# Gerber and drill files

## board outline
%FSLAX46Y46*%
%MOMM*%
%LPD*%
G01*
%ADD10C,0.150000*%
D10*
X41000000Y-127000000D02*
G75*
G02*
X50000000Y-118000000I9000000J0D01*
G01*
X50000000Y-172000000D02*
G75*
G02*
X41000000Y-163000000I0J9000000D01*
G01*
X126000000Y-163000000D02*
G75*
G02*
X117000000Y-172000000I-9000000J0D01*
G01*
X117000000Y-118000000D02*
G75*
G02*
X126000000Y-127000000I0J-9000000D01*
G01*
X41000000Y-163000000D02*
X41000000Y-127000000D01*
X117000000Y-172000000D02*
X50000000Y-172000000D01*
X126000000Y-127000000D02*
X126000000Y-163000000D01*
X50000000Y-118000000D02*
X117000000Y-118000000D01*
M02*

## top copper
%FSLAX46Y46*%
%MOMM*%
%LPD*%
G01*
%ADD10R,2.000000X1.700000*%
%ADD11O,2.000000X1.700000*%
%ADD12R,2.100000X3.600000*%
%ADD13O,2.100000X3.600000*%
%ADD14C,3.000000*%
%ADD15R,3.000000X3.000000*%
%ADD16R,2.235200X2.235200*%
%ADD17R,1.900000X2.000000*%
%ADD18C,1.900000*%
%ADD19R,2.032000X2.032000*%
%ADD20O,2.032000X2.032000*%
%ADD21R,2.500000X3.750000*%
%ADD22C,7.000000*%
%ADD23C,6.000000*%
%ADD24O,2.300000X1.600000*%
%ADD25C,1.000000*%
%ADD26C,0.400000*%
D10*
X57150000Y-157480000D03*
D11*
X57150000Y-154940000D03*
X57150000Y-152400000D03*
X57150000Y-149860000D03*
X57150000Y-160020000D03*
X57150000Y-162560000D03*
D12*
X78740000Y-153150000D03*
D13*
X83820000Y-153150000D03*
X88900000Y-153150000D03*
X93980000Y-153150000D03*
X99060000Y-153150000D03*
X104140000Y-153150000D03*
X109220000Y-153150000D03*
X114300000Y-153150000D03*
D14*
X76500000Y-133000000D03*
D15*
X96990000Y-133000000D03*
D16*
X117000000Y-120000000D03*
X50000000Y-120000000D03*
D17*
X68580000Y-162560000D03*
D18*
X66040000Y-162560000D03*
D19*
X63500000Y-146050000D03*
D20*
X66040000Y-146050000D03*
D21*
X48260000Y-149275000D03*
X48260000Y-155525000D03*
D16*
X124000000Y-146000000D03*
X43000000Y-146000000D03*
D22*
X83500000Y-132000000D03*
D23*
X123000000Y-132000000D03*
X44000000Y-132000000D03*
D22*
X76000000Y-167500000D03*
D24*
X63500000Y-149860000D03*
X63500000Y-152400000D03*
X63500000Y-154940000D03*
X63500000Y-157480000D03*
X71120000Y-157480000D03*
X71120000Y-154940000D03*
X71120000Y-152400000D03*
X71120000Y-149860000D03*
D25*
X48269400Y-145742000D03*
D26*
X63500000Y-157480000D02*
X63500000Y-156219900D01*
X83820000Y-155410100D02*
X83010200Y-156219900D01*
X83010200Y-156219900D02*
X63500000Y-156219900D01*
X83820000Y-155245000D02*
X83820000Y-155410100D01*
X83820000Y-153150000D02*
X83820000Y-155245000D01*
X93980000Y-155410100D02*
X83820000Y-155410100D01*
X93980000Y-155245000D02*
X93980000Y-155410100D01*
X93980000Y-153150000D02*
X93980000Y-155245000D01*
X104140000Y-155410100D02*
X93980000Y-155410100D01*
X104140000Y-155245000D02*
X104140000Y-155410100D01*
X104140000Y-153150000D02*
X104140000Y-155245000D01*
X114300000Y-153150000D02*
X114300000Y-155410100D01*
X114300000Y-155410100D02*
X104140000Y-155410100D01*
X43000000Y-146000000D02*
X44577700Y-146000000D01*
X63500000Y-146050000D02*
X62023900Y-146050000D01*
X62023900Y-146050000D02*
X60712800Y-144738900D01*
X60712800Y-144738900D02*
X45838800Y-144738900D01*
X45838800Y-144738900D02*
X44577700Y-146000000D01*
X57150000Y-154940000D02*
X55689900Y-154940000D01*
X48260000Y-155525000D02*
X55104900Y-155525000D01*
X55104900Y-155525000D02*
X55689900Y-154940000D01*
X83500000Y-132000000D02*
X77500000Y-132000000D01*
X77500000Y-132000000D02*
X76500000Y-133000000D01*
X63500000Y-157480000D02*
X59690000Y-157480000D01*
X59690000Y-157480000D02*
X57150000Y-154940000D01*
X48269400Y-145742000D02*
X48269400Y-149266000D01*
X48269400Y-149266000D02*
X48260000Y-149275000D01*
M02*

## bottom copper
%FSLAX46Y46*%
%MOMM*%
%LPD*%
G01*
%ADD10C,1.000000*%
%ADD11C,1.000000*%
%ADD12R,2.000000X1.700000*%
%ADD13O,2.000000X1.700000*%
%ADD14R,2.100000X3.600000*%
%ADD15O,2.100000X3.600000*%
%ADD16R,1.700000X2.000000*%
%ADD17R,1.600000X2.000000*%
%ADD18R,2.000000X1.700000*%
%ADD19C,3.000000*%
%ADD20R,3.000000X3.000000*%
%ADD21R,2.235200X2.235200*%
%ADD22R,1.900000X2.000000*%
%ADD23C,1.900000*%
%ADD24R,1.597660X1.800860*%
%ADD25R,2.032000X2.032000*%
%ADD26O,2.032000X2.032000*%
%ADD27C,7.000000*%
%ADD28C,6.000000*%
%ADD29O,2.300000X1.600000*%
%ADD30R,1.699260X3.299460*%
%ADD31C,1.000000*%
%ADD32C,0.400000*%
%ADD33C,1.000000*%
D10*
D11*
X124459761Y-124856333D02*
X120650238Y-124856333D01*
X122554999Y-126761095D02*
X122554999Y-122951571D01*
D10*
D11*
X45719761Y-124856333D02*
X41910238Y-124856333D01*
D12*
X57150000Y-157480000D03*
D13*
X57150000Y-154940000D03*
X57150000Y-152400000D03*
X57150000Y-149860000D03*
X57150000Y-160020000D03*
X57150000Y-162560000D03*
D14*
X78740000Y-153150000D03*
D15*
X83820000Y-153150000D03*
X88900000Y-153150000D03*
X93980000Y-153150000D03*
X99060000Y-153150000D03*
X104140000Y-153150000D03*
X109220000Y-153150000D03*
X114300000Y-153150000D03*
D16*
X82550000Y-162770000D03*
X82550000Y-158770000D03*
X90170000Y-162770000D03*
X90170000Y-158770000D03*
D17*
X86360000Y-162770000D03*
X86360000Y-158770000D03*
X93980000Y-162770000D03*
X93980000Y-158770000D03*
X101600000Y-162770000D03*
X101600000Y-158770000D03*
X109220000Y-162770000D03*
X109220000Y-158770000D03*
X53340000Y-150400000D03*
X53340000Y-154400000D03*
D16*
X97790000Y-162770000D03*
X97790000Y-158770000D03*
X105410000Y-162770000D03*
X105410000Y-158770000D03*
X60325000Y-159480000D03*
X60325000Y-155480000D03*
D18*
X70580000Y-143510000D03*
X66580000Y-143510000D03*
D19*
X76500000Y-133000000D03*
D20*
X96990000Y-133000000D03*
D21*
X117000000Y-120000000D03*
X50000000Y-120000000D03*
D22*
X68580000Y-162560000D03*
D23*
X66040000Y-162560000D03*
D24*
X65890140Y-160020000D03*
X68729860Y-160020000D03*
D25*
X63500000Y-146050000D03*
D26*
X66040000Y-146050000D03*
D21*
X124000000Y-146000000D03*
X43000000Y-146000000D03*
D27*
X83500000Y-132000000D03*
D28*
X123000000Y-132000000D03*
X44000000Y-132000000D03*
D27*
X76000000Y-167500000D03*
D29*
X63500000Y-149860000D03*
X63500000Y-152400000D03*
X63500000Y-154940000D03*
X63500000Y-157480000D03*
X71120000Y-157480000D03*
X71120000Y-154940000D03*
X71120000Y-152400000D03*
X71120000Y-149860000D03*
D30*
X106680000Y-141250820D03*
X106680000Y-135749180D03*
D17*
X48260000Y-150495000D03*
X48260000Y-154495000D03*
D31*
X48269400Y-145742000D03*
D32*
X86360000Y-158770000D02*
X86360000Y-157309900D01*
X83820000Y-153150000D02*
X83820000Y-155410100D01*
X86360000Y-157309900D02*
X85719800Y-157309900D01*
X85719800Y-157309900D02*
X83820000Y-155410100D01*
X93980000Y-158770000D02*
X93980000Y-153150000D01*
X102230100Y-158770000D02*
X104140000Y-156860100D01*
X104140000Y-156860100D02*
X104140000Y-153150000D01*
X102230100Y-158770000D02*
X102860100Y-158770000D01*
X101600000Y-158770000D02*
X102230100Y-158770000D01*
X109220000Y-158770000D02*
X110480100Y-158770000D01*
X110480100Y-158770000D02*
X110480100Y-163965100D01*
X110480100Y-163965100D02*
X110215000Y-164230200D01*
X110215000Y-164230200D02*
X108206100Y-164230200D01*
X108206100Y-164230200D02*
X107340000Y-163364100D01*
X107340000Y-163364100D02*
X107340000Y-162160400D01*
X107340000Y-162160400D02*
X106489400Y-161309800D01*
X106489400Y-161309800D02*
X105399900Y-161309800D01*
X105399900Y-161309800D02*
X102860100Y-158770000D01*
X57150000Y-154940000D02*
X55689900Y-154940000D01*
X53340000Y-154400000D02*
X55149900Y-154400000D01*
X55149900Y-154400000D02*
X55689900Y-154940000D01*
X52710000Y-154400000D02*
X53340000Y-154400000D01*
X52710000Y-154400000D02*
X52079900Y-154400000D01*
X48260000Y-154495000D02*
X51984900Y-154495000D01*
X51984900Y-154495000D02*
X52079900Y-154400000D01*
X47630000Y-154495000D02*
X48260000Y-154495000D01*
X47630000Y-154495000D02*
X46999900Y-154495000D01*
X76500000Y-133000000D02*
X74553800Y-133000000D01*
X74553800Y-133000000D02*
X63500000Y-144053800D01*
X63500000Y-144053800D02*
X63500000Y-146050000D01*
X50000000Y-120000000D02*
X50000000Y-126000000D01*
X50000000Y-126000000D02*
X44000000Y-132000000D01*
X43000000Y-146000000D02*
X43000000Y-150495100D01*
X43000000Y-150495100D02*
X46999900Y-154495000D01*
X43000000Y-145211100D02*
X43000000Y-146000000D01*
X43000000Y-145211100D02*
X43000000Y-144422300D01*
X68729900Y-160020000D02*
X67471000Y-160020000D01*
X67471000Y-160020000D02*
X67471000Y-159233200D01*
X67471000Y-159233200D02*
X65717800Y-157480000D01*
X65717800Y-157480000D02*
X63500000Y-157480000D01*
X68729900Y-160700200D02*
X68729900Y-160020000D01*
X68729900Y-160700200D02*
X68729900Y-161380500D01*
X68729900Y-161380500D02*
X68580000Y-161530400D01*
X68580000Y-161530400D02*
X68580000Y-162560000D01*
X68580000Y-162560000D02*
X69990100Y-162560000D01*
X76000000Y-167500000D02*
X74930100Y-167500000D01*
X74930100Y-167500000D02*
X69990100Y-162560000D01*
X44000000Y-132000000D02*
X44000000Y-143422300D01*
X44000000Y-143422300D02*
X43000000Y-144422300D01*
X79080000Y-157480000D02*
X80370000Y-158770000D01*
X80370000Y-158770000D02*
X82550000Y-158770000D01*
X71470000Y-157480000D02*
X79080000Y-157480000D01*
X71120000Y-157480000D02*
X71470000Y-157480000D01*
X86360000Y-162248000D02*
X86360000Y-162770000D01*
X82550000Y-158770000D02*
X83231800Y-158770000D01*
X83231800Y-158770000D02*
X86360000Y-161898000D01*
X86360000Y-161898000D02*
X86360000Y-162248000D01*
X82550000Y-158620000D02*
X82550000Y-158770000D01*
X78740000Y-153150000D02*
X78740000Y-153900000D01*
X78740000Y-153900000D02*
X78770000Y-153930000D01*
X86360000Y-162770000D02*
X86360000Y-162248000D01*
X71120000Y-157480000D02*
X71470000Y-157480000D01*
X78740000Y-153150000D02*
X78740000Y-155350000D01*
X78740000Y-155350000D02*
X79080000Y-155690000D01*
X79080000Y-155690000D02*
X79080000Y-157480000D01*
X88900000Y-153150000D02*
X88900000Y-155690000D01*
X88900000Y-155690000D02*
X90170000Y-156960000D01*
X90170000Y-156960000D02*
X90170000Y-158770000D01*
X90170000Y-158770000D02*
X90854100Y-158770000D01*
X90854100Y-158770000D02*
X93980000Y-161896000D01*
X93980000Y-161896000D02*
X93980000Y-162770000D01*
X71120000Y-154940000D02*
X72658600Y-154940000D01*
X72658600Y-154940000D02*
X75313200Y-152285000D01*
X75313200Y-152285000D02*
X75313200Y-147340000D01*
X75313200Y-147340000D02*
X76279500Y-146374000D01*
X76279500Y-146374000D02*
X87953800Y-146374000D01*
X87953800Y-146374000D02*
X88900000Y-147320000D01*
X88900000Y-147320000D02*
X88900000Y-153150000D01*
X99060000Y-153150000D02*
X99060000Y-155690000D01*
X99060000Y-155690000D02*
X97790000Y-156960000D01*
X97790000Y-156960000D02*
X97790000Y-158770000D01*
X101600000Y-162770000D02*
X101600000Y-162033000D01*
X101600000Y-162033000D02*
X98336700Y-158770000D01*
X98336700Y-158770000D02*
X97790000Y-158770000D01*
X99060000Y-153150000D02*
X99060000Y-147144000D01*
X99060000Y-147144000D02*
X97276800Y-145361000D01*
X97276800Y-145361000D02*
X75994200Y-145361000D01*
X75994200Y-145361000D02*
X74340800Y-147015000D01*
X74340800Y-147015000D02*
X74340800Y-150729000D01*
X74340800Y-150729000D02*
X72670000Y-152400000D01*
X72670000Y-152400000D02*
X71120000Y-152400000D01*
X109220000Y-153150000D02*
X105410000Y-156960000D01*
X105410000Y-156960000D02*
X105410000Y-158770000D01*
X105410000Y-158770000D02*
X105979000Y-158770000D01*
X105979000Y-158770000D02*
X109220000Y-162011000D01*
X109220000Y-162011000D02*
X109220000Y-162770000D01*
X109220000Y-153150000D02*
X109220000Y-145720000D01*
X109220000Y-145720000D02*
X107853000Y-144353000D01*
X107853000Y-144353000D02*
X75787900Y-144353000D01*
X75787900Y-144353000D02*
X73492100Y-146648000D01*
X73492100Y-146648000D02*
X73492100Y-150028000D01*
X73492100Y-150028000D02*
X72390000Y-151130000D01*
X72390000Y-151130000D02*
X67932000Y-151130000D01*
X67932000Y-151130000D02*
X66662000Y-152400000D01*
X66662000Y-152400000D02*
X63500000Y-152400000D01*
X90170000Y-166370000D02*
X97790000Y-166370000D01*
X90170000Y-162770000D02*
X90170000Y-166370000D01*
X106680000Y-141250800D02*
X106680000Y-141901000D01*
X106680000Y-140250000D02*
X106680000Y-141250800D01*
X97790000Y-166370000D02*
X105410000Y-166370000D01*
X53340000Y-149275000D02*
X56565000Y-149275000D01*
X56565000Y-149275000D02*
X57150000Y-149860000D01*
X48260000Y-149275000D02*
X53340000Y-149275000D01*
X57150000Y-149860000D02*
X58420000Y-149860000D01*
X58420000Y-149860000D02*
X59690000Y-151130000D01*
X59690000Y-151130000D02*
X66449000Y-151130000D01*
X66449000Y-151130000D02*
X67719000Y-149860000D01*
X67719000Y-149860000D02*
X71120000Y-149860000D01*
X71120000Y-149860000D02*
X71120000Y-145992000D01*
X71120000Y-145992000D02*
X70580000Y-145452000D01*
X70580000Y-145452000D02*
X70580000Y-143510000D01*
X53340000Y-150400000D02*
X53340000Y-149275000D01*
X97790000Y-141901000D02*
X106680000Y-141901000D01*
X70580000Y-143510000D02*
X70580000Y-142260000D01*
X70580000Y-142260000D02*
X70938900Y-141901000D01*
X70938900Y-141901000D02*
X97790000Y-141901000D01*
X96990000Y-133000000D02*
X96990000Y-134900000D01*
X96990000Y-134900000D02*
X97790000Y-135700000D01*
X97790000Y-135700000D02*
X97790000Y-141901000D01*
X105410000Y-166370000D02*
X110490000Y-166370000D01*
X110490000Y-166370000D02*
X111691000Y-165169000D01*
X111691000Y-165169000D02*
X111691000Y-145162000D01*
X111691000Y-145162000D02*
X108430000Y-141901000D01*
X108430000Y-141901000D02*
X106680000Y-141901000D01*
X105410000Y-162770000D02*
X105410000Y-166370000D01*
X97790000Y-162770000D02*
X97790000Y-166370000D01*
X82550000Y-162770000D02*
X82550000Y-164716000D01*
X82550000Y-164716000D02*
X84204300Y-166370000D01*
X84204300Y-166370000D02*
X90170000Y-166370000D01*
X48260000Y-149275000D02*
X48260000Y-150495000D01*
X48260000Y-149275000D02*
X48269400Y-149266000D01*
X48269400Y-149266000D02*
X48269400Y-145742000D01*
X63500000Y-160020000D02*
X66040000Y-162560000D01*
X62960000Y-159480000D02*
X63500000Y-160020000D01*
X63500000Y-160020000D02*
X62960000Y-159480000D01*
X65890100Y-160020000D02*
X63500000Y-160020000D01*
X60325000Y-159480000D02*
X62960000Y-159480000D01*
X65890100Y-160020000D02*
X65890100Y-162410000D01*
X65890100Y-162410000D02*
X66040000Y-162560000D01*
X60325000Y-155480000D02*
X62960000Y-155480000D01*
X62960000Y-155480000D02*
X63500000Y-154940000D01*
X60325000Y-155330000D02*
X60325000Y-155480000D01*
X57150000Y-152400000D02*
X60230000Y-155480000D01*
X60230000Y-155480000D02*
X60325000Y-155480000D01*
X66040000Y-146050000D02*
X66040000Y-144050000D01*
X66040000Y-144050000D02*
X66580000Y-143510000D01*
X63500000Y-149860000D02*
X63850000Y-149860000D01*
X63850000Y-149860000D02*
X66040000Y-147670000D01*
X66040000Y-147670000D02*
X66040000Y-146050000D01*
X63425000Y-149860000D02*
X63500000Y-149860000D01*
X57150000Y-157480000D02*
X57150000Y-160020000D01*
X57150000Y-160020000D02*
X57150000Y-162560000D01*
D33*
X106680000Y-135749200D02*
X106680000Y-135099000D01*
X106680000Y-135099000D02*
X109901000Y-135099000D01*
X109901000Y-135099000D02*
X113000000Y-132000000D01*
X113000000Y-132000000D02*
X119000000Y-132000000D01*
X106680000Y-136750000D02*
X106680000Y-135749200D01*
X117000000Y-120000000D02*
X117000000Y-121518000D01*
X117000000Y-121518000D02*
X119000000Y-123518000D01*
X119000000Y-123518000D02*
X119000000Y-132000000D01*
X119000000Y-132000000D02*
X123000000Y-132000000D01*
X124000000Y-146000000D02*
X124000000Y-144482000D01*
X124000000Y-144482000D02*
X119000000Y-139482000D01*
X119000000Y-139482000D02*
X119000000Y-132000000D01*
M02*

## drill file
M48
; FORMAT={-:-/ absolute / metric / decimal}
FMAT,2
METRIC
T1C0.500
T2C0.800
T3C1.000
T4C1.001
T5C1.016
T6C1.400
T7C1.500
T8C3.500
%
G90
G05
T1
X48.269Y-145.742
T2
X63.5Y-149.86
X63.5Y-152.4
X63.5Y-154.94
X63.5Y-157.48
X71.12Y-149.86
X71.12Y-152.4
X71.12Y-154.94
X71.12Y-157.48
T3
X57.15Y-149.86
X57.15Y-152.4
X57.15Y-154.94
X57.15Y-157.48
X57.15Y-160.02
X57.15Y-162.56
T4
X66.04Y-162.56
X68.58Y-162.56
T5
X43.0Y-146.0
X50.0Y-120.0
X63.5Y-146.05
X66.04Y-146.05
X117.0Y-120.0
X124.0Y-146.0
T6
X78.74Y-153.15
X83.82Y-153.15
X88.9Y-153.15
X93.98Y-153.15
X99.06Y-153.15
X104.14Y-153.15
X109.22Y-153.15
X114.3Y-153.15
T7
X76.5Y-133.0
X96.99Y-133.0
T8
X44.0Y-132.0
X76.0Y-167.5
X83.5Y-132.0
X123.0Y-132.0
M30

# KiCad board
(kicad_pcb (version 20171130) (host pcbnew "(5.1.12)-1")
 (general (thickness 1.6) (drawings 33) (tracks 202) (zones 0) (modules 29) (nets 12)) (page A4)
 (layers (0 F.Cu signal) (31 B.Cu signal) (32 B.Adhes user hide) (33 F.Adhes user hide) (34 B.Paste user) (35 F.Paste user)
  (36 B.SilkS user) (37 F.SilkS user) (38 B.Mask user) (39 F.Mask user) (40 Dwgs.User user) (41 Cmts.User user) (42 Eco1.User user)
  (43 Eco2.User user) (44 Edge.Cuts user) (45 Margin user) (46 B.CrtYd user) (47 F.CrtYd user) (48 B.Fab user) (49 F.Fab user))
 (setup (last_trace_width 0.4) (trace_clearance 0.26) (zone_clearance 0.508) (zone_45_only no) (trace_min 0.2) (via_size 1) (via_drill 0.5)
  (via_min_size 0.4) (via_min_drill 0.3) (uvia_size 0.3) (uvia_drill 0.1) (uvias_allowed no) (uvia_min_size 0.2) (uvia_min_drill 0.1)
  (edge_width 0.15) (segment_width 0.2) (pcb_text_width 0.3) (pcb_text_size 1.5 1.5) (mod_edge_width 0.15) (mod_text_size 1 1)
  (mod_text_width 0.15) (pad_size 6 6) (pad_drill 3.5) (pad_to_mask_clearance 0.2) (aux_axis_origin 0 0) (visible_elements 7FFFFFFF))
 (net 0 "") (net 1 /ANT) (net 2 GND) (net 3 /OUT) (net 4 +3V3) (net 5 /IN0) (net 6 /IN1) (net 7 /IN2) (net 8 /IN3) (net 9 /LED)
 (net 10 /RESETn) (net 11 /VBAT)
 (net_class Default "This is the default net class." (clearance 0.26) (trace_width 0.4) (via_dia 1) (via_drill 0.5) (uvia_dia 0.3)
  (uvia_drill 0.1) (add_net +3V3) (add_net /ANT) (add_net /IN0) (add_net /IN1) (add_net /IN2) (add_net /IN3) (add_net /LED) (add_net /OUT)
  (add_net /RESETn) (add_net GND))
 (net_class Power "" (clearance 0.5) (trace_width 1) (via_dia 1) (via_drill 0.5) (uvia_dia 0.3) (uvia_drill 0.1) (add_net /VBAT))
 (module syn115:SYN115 (layer F.Cu) (at 57.15 154.94 180)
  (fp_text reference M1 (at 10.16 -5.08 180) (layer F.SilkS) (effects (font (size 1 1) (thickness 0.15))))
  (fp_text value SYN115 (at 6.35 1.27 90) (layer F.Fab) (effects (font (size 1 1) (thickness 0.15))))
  (pad 1 thru_hole rect (at 0 -2.54 180) (size 2 1.7) (drill 1) (layers *.Cu *.Mask) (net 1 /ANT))
  (pad 2 thru_hole oval (at 0 0 180) (size 2 1.7) (drill 1) (layers *.Cu *.Mask) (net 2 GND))
  (pad 3 thru_hole oval (at 0 2.54 180) (size 2 1.7) (drill 1) (layers *.Cu *.Mask) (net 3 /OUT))
  (pad 4 thru_hole oval (at 0 5.08 180) (size 2 1.7) (drill 1) (layers *.Cu *.Mask) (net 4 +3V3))
  (pad 1 thru_hole oval (at 0 -5.08 180) (size 2 1.7) (drill 1) (layers *.Cu *.Mask) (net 1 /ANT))
  (pad 1 thru_hole oval (at 0 -7.62 180) (size 2 1.7) (drill 1) (layers *.Cu *.Mask) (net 1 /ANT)))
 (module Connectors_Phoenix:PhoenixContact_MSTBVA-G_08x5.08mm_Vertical (layer F.Cu) (at 78.74 153.15)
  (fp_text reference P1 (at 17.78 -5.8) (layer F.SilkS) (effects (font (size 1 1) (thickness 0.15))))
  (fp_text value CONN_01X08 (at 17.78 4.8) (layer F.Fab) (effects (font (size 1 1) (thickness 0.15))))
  (pad 1 thru_hole rect (at 0 0) (size 2.1 3.6) (drill 1.4) (layers *.Cu *.Mask) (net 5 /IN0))
  (pad 2 thru_hole oval (at 5.08 0) (size 2.1 3.6) (drill 1.4) (layers *.Cu *.Mask) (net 2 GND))
  (pad 3 thru_hole oval (at 10.16 0) (size 2.1 3.6) (drill 1.4) (layers *.Cu *.Mask) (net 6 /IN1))
  (pad 4 thru_hole oval (at 15.24 0) (size 2.1 3.6) (drill 1.4) (layers *.Cu *.Mask) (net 2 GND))
  (pad 5 thru_hole oval (at 20.32 0) (size 2.1 3.6) (drill 1.4) (layers *.Cu *.Mask) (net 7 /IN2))
  (pad 6 thru_hole oval (at 25.4 0) (size 2.1 3.6) (drill 1.4) (layers *.Cu *.Mask) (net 2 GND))
  (pad 7 thru_hole oval (at 30.48 0) (size 2.1 3.6) (drill 1.4) (layers *.Cu *.Mask) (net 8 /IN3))
  (pad 8 thru_hole oval (at 35.56 0) (size 2.1 3.6) (drill 1.4) (layers *.Cu *.Mask) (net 2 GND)))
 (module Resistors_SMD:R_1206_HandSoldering (layer B.Cu) (at 82.55 160.77 90)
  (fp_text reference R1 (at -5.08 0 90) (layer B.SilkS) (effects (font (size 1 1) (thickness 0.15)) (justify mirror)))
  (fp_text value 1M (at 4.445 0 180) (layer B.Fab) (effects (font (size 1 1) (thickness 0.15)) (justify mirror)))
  (pad 1 smd rect (at -2 0 90) (size 2 1.7) (layers B.Cu B.Paste B.Mask) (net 4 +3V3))
  (pad 2 smd rect (at 2 0 90) (size 2 1.7) (layers B.Cu B.Paste B.Mask) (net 5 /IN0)))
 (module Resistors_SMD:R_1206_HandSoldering (layer B.Cu) (at 90.17 160.77 90)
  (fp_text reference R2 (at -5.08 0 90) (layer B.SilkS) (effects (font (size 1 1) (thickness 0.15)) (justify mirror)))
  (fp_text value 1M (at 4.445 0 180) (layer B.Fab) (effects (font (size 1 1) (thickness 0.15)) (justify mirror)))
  (pad 1 smd rect (at -2 0 90) (size 2 1.7) (layers B.Cu B.Paste B.Mask) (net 4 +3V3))
  (pad 2 smd rect (at 2 0 90) (size 2 1.7) (layers B.Cu B.Paste B.Mask) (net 6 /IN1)))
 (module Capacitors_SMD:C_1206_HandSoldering (layer B.Cu) (at 86.36 160.77 90)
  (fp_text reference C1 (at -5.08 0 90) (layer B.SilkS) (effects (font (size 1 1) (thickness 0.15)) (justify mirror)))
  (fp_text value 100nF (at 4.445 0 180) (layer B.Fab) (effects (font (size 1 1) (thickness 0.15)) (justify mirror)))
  (pad 1 smd rect (at -2 0 90) (size 2 1.6) (layers B.Cu B.Paste B.Mask) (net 5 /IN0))
  (pad 2 smd rect (at 2 0 90) (size 2 1.6) (layers B.Cu B.Paste B.Mask) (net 2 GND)))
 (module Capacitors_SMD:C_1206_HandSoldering (layer B.Cu) (at 93.98 160.77 90)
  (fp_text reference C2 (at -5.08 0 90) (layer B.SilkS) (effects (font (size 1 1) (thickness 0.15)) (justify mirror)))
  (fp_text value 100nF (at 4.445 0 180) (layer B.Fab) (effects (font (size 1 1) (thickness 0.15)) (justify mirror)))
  (pad 1 smd rect (at -2 0 90) (size 2 1.6) (layers B.Cu B.Paste B.Mask) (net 6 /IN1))
  (pad 2 smd rect (at 2 0 90) (size 2 1.6) (layers B.Cu B.Paste B.Mask) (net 2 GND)))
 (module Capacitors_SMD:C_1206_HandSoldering (layer B.Cu) (at 101.6 160.77 90)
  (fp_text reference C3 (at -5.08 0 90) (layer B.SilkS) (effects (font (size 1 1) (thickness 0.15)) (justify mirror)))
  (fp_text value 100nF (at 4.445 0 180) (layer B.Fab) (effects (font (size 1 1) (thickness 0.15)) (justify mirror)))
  (pad 1 smd rect (at -2 0 90) (size 2 1.6) (layers B.Cu B.Paste B.Mask) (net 7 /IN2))
  (pad 2 smd rect (at 2 0 90) (size 2 1.6) (layers B.Cu B.Paste B.Mask) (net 2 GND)))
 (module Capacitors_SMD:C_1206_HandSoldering (layer B.Cu) (at 109.22 160.77 90)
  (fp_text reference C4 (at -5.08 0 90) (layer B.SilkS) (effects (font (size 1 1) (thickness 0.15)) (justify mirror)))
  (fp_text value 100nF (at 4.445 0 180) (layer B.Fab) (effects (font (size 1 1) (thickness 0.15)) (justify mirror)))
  (pad 1 smd rect (at -2 0 90) (size 2 1.6) (layers B.Cu B.Paste B.Mask) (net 8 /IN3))
  (pad 2 smd rect (at 2 0 90) (size 2 1.6) (layers B.Cu B.Paste B.Mask) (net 2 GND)))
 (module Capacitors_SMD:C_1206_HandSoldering (layer B.Cu) (at 53.34 152.4 270)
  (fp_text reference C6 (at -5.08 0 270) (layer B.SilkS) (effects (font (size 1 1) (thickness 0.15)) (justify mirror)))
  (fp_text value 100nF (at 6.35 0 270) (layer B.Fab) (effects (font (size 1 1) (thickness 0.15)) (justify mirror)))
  (pad 1 smd rect (at -2 0 270) (size 2 1.6) (layers B.Cu B.Paste B.Mask) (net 4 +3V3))
  (pad 2 smd rect (at 2 0 270) (size 2 1.6) (layers B.Cu B.Paste B.Mask) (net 2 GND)))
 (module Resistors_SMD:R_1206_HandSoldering (layer B.Cu) (at 97.79 160.77 90)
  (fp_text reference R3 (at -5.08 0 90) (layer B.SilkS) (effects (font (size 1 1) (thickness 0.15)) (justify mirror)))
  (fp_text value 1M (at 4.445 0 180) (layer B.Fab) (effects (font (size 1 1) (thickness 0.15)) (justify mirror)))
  (pad 1 smd rect (at -2 0 90) (size 2 1.7) (layers B.Cu B.Paste B.Mask) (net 4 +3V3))
  (pad 2 smd rect (at 2 0 90) (size 2 1.7) (layers B.Cu B.Paste B.Mask) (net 7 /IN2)))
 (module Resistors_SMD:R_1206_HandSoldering (layer B.Cu) (at 105.41 160.77 90)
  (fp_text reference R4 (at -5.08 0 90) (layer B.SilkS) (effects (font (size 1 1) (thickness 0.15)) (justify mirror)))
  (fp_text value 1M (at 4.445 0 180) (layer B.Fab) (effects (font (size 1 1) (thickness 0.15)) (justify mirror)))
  (pad 1 smd rect (at -2 0 90) (size 2 1.7) (layers B.Cu B.Paste B.Mask) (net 4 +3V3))
  (pad 2 smd rect (at 2 0 90) (size 2 1.7) (layers B.Cu B.Paste B.Mask) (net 8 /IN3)))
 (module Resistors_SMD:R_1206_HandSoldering (layer B.Cu) (at 60.325 157.48 90)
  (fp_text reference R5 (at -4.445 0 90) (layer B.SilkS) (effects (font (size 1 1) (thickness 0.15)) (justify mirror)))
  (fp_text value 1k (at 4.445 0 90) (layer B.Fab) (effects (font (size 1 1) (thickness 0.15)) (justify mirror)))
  (pad 1 smd rect (at -2 0 90) (size 2 1.7) (layers B.Cu B.Paste B.Mask) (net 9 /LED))
  (pad 2 smd rect (at 2 0 90) (size 2 1.7) (layers B.Cu B.Paste B.Mask) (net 3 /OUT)))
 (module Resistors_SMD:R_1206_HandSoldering (layer B.Cu) (at 68.58 143.51 180)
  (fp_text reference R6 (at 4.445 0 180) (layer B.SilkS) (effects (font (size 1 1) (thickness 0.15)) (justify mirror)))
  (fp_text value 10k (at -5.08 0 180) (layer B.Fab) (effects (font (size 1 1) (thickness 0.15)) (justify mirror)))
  (pad 1 smd rect (at -2 0 180) (size 2 1.7) (layers B.Cu B.Paste B.Mask) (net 4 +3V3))
  (pad 2 smd rect (at 2 0 180) (size 2 1.7) (layers B.Cu B.Paste B.Mask) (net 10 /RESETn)))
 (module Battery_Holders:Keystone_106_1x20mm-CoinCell (layer F.Cu) (at 96.99 133 180)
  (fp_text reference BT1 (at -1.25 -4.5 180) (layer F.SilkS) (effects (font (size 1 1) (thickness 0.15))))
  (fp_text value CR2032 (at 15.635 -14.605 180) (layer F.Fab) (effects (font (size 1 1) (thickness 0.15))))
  (pad 2 thru_hole circle (at 20.49 0 180) (size 3 3) (drill 1.5) (layers *.Cu *.Mask) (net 2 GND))
  (pad 1 thru_hole rect (at 0 0 180) (size 3 3) (drill 1.5) (layers *.Cu *.Mask) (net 4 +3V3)))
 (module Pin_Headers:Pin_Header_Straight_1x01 (layer F.Cu) (at 117 120)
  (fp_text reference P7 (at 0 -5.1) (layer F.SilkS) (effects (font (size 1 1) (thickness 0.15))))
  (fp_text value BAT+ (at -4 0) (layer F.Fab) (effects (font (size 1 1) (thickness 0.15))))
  (pad 1 thru_hole rect (at 0 0) (size 2.2352 2.2352) (drill 1.016) (layers *.Cu *.Mask) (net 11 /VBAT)))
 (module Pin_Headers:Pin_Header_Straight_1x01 (layer F.Cu) (at 50 120)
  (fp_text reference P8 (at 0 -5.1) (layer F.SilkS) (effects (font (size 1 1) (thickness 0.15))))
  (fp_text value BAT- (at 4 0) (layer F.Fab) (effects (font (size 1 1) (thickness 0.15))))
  (pad 1 thru_hole rect (at 0 0) (size 2.2352 2.2352) (drill 1.016) (layers *.Cu *.Mask) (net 2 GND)))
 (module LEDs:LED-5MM (layer F.Cu) (at 68.58 162.56 180)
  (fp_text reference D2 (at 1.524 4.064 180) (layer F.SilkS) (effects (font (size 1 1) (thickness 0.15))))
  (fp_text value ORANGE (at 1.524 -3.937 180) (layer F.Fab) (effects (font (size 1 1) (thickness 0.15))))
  (pad 1 thru_hole rect (at 0 0 270) (size 2 1.9) (drill 1.00076) (layers *.Cu *.Mask) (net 2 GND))
  (pad 2 thru_hole circle (at 2.54 0 180) (size 1.9 1.9) (drill 1.00076) (layers *.Cu *.Mask) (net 9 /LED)))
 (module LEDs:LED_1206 (layer B.Cu) (at 67.31 160.02 180)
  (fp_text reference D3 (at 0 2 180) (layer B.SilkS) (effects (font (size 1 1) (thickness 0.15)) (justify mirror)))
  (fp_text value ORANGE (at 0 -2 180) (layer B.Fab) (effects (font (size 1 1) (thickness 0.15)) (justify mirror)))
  (pad 2 smd rect (at 1.41986 0) (size 1.59766 1.80086) (layers B.Cu B.Paste B.Mask) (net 9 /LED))
  (pad 1 smd rect (at -1.41986 0) (size 1.59766 1.80086) (layers B.Cu B.Paste B.Mask) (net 2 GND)))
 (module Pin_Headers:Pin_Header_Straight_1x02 (layer F.Cu) (at 63.5 146.05 90)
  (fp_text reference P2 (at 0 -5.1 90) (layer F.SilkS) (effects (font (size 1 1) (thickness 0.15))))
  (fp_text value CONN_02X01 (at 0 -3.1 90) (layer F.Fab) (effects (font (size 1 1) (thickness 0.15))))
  (pad 1 thru_hole rect (at 0 0 90) (size 2.032 2.032) (drill 1.016) (layers *.Cu *.Mask) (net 2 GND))
  (pad 2 thru_hole oval (at 0 2.54 90) (size 2.032 2.032) (drill 1.016) (layers *.Cu *.Mask) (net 10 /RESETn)))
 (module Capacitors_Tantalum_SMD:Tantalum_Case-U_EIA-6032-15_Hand (layer F.Cu) (at 48.26 152.4 270)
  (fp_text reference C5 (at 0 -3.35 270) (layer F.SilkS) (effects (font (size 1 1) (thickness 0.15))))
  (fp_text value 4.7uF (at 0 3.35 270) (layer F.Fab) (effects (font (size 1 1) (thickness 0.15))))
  (pad 1 smd rect (at -3.125 0 270) (size 3.75 2.5) (layers F.Cu F.Paste F.Mask) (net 4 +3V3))
  (pad 2 smd rect (at 3.125 0 270) (size 3.75 2.5) (layers F.Cu F.Paste F.Mask) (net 2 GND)))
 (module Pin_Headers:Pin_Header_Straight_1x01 (layer F.Cu) (at 124 146)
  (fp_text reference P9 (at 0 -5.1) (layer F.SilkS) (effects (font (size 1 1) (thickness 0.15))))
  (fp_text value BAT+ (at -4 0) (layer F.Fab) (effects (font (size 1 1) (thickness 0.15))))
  (pad 1 thru_hole rect (at 0 0) (size 2.2352 2.2352) (drill 1.016) (layers *.Cu *.Mask) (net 11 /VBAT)))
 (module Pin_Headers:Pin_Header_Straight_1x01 (layer F.Cu) (at 43 146)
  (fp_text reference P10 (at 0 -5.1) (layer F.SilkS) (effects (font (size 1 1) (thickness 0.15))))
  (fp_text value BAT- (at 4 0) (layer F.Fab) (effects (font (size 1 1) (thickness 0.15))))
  (pad 1 thru_hole rect (at 0 0) (size 2.2352 2.2352) (drill 1.016) (layers *.Cu *.Mask) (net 2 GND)))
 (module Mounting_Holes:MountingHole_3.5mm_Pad (layer F.Cu) (at 83.5 132)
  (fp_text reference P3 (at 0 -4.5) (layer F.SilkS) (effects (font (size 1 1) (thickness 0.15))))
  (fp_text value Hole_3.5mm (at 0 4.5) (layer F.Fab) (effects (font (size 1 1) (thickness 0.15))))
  (pad 1 thru_hole circle (at 0 0) (size 7 7) (drill 3.5) (layers *.Cu *.Mask) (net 2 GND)))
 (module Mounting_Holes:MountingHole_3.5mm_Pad (layer F.Cu) (at 123 132)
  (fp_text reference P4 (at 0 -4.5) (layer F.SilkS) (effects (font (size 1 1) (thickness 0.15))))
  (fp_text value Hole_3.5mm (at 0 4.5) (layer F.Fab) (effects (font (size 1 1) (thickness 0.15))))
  (pad 1 thru_hole circle (at 0 0) (size 6 6) (drill 3.5) (layers *.Cu *.Mask) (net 11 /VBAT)))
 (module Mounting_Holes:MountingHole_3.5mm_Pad (layer F.Cu) (at 44 132)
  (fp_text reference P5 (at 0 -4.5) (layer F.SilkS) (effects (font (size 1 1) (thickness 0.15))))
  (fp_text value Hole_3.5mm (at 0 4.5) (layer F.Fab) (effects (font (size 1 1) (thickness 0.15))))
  (pad 1 thru_hole circle (at 0 0) (size 6 6) (drill 3.5) (layers *.Cu *.Mask) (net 2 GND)))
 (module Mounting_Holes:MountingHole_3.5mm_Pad (layer F.Cu) (at 76 167.5)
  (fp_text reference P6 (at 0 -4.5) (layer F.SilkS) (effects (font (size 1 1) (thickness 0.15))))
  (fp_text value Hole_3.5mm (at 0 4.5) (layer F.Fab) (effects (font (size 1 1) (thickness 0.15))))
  (pad 1 thru_hole circle (at 0 0) (size 7 7) (drill 3.5) (layers *.Cu *.Mask) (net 2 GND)))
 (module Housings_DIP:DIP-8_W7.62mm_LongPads (layer F.Cu) (at 63.5 149.86)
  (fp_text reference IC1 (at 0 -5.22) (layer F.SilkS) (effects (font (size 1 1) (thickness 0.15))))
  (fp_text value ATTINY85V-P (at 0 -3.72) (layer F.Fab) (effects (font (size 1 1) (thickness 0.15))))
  (pad 1 thru_hole oval (at 0 0) (size 2.3 1.6) (drill 0.8) (layers *.Cu *.Mask) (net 10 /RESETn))
  (pad 2 thru_hole oval (at 0 2.54) (size 2.3 1.6) (drill 0.8) (layers *.Cu *.Mask) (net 8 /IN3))
  (pad 3 thru_hole oval (at 0 5.08) (size 2.3 1.6) (drill 0.8) (layers *.Cu *.Mask) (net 3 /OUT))
  (pad 4 thru_hole oval (at 0 7.62) (size 2.3 1.6) (drill 0.8) (layers *.Cu *.Mask) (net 2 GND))
  (pad 5 thru_hole oval (at 7.62 7.62) (size 2.3 1.6) (drill 0.8) (layers *.Cu *.Mask) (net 5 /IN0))
  (pad 6 thru_hole oval (at 7.62 5.08) (size 2.3 1.6) (drill 0.8) (layers *.Cu *.Mask) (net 6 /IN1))
  (pad 7 thru_hole oval (at 7.62 2.54) (size 2.3 1.6) (drill 0.8) (layers *.Cu *.Mask) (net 7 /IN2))
  (pad 8 thru_hole oval (at 7.62 0) (size 2.3 1.6) (drill 0.8) (layers *.Cu *.Mask) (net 4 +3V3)))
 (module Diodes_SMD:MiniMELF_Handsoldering (layer B.Cu) (at 106.68 138.5 90)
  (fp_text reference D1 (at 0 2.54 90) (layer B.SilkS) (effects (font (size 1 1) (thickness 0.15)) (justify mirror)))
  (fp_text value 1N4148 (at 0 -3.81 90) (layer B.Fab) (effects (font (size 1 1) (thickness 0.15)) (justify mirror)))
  (pad 1 smd rect (at -2.75082 0 90) (size 3.29946 1.69926) (layers B.Cu B.Paste B.Mask) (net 4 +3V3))
  (pad 2 smd rect (at 2.75082 0 90) (size 3.29946 1.69926) (layers B.Cu B.Paste B.Mask) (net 11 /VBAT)))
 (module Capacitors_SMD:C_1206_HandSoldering (layer B.Cu) (at 48.26 152.495 270)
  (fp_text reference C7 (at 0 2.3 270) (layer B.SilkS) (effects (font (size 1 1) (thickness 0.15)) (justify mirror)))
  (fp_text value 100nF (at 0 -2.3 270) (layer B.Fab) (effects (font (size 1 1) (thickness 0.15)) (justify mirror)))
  (pad 1 smd rect (at -2 0 270) (size 2 1.6) (layers B.Cu B.Paste B.Mask) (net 4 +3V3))
  (pad 2 smd rect (at 2 0 270) (size 2 1.6) (layers B.Cu B.Paste B.Mask) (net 2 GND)))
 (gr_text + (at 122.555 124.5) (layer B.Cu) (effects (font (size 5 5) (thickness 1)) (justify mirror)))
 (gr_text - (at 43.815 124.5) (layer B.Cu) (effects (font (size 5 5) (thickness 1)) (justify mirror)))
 (gr_arc (start 50 127) (end 41 127) (angle 90) (layer Edge.Cuts) (width 0.15))
 (gr_arc (start 50 163) (end 50 172) (angle 90) (layer Edge.Cuts) (width 0.15))
 (gr_arc (start 117 163) (end 126 163) (angle 90) (layer Edge.Cuts) (width 0.15))
 (gr_arc (start 117 127) (end 117 118) (angle 90) (layer Edge.Cuts) (width 0.15))
 (gr_line (start 41 163) (end 41 127) (layer Edge.Cuts) (width 0.15))
 (gr_line (start 117 172) (end 50 172) (layer Edge.Cuts) (width 0.15))
 (gr_line (start 126 127) (end 126 163) (layer Edge.Cuts) (width 0.15))
 (gr_line (start 50 118) (end 117 118) (layer Edge.Cuts) (width 0.15))
 (segment (start 63.5 157.48) (end 63.5 156.2199) (width 0.4) (layer F.Cu) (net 2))
 (segment (start 83.82 155.4101) (end 83.0102 156.2199) (width 0.4) (layer F.Cu) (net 2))
 (segment (start 83.0102 156.2199) (end 63.5 156.2199) (width 0.4) (layer F.Cu) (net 2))
 (segment (start 83.82 155.245) (end 83.82 155.4101) (width 0.4) (layer F.Cu) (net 2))
 (segment (start 83.82 153.15) (end 83.82 155.245) (width 0.4) (layer F.Cu) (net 2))
 (segment (start 93.98 155.4101) (end 83.82 155.4101) (width 0.4) (layer F.Cu) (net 2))
 (segment (start 93.98 155.245) (end 93.98 155.4101) (width 0.4) (layer F.Cu) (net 2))
 (segment (start 93.98 153.15) (end 93.98 155.245) (width 0.4) (layer F.Cu) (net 2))
 (segment (start 104.14 155.4101) (end 93.98 155.4101) (width 0.4) (layer F.Cu) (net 2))
 (segment (start 104.14 155.245) (end 104.14 155.4101) (width 0.4) (layer F.Cu) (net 2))
 (segment (start 104.14 153.15) (end 104.14 155.245) (width 0.4) (layer F.Cu) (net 2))
 (segment (start 114.3 153.15) (end 114.3 155.4101) (width 0.4) (layer F.Cu) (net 2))
 (segment (start 114.3 155.4101) (end 104.14 155.4101) (width 0.4) (layer F.Cu) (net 2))
 (segment (start 86.36 158.77) (end 86.36 157.3099) (width 0.4) (layer B.Cu) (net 2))
 (segment (start 83.82 153.15) (end 83.82 155.4101) (width 0.4) (layer B.Cu) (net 2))
 (segment (start 86.36 157.3099) (end 85.7198 157.3099) (width 0.4) (layer B.Cu) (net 2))
 (segment (start 85.7198 157.3099) (end 83.82 155.4101) (width 0.4) (layer B.Cu) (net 2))
 (segment (start 93.98 158.77) (end 93.98 153.15) (width 0.4) (layer B.Cu) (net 2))
 (segment (start 102.2301 158.77) (end 104.14 156.8601) (width 0.4) (layer B.Cu) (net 2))
 (segment (start 104.14 156.8601) (end 104.14 153.15) (width 0.4) (layer B.Cu) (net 2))
 (segment (start 102.2301 158.77) (end 102.8601 158.77) (width 0.4) (layer B.Cu) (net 2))
 (segment (start 101.6 158.77) (end 102.2301 158.77) (width 0.4) (layer B.Cu) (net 2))
 (segment (start 109.22 158.77) (end 110.4801 158.77) (width 0.4) (layer B.Cu) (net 2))
 (segment (start 110.4801 158.77) (end 110.4801 163.9651) (width 0.4) (layer B.Cu) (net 2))
 (segment (start 110.4801 163.9651) (end 110.215 164.2302) (width 0.4) (layer B.Cu) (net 2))
 (segment (start 110.215 164.2302) (end 108.2061 164.2302) (width 0.4) (layer B.Cu) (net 2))
 (segment (start 108.2061 164.2302) (end 107.34 163.3641) (width 0.4) (layer B.Cu) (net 2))
 (segment (start 107.34 163.3641) (end 107.34 162.1604) (width 0.4) (layer B.Cu) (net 2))
 (segment (start 107.34 162.1604) (end 106.4894 161.3098) (width 0.4) (layer B.Cu) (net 2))
 (segment (start 106.4894 161.3098) (end 105.3999 161.3098) (width 0.4) (layer B.Cu) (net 2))
 (segment (start 105.3999 161.3098) (end 102.8601 158.77) (width 0.4) (layer B.Cu) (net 2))
 (segment (start 57.15 154.94) (end 55.6899 154.94) (width 0.4) (layer B.Cu) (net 2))
 (segment (start 53.34 154.4) (end 55.1499 154.4) (width 0.4) (layer B.Cu) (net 2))
 (segment (start 55.1499 154.4) (end 55.6899 154.94) (width 0.4) (layer B.Cu) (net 2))
 (segment (start 52.71 154.4) (end 53.34 154.4) (width 0.4) (layer B.Cu) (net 2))
 (segment (start 52.71 154.4) (end 52.0799 154.4) (width 0.4) (layer B.Cu) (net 2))
 (segment (start 48.26 154.495) (end 51.9849 154.495) (width 0.4) (layer B.Cu) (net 2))
 (segment (start 51.9849 154.495) (end 52.0799 154.4) (width 0.4) (layer B.Cu) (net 2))
 (segment (start 47.63 154.495) (end 48.26 154.495) (width 0.4) (layer B.Cu) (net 2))
 (segment (start 47.63 154.495) (end 46.9999 154.495) (width 0.4) (layer B.Cu) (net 2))
 (segment (start 76.5 133) (end 74.5538 133) (width 0.4) (layer B.Cu) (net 2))
 (segment (start 74.5538 133) (end 63.5 144.0538) (width 0.4) (layer B.Cu) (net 2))
 (segment (start 63.5 144.0538) (end 63.5 146.05) (width 0.4) (layer B.Cu) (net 2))
 (segment (start 50 120) (end 50 126) (width 0.4) (layer B.Cu) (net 2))
 (segment (start 50 126) (end 44 132) (width 0.4) (layer B.Cu) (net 2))
 (segment (start 43 146) (end 43 150.4951) (width 0.4) (layer B.Cu) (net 2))
 (segment (start 43 150.4951) (end 46.9999 154.495) (width 0.4) (layer B.Cu) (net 2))
 (segment (start 43 145.2111) (end 43 146) (width 0.4) (layer B.Cu) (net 2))
 (segment (start 43 145.2111) (end 43 144.4223) (width 0.4) (layer B.Cu) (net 2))
 (segment (start 68.7299 160.02) (end 67.471 160.02) (width 0.4) (layer B.Cu) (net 2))
 (segment (start 67.471 160.02) (end 67.471 159.2332) (width 0.4) (layer B.Cu) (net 2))
 (segment (start 67.471 159.2332) (end 65.7178 157.48) (width 0.4) (layer B.Cu) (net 2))
 (segment (start 65.7178 157.48) (end 63.5 157.48) (width 0.4) (layer B.Cu) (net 2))
 (segment (start 68.7299 160.7002) (end 68.7299 160.02) (width 0.4) (layer B.Cu) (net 2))
 (segment (start 68.7299 160.7002) (end 68.7299 161.3805) (width 0.4) (layer B.Cu) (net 2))
 (segment (start 68.7299 161.3805) (end 68.58 161.5304) (width 0.4) (layer B.Cu) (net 2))
 (segment (start 68.58 161.5304) (end 68.58 162.56) (width 0.4) (layer B.Cu) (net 2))
 (segment (start 43 146) (end 44.5777 146) (width 0.4) (layer F.Cu) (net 2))
 (segment (start 63.5 146.05) (end 62.0239 146.05) (width 0.4) (layer F.Cu) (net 2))
 (segment (start 62.0239 146.05) (end 60.7128 144.7389) (width 0.4) (layer F.Cu) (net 2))
 (segment (start 60.7128 144.7389) (end 45.8388 144.7389) (width 0.4) (layer F.Cu) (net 2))
 (segment (start 45.8388 144.7389) (end 44.5777 146) (width 0.4) (layer F.Cu) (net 2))
 (segment (start 57.15 154.94) (end 55.6899 154.94) (width 0.4) (layer F.Cu) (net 2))
 (segment (start 48.26 155.525) (end 55.1049 155.525) (width 0.4) (layer F.Cu) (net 2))
 (segment (start 55.1049 155.525) (end 55.6899 154.94) (width 0.4) (layer F.Cu) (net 2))
 (segment (start 83.5 132) (end 77.5 132) (width 0.4) (layer F.Cu) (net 2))
 (segment (start 77.5 132) (end 76.5 133) (width 0.4) (layer F.Cu) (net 2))
 (segment (start 68.58 162.56) (end 69.9901 162.56) (width 0.4) (layer B.Cu) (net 2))
 (segment (start 76 167.5) (end 74.9301 167.5) (width 0.4) (layer B.Cu) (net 2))
 (segment (start 74.9301 167.5) (end 69.9901 162.56) (width 0.4) (layer B.Cu) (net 2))
 (segment (start 44 132) (end 44 143.4223) (width 0.4) (layer B.Cu) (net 2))
 (segment (start 44 143.4223) (end 43 144.4223) (width 0.4) (layer B.Cu) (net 2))
 (segment (start 63.5 157.48) (end 59.69 157.48) (width 0.4) (layer F.Cu) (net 2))
 (segment (start 59.69 157.48) (end 57.15 154.94) (width 0.4) (layer F.Cu) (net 2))
 (segment (start 79.08 157.48) (end 80.37 158.77) (width 0.4) (layer B.Cu) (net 5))
 (segment (start 80.37 158.77) (end 82.55 158.77) (width 0.4) (layer B.Cu) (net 5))
 (segment (start 71.47 157.48) (end 79.08 157.48) (width 0.4) (layer B.Cu) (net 5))
 (segment (start 71.12 157.48) (end 71.47 157.48) (width 0.4) (layer B.Cu) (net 5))
 (segment (start 86.36 162.248) (end 86.36 162.77) (width 0.4) (layer B.Cu) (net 5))
 (segment (start 82.55 158.77) (end 83.2318 158.77) (width 0.4) (layer B.Cu) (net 5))
 (segment (start 83.2318 158.77) (end 86.36 161.898) (width 0.4) (layer B.Cu) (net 5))
 (segment (start 86.36 161.898) (end 86.36 162.248) (width 0.4) (layer B.Cu) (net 5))
 (segment (start 82.55 158.62) (end 82.55 158.77) (width 0.4) (layer B.Cu) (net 5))
 (segment (start 78.74 153.15) (end 78.74 153.9) (width 0.4) (layer B.Cu) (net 5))
 (segment (start 78.74 153.9) (end 78.77 153.93) (width 0.4) (layer B.Cu) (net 5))
 (segment (start 86.36 162.77) (end 86.36 162.248) (width 0.4) (layer B.Cu) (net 5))
 (segment (start 71.12 157.48) (end 71.47 157.48) (width 0.4) (layer B.Cu) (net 5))
 (segment (start 78.74 153.15) (end 78.74 155.35) (width 0.4) (layer B.Cu) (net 5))
 (segment (start 78.74 155.35) (end 79.08 155.69) (width 0.4) (layer B.Cu) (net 5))
 (segment (start 79.08 155.69) (end 79.08 157.48) (width 0.4) (layer B.Cu) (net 5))
 (segment (start 88.9 153.15) (end 88.9 155.69) (width 0.4) (layer B.Cu) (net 6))
 (segment (start 88.9 155.69) (end 90.17 156.96) (width 0.4) (layer B.Cu) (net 6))
 (segment (start 90.17 156.96) (end 90.17 158.77) (width 0.4) (layer B.Cu) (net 6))
 (segment (start 90.17 158.77) (end 90.8541 158.77) (width 0.4) (layer B.Cu) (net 6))
 (segment (start 90.8541 158.77) (end 93.98 161.896) (width 0.4) (layer B.Cu) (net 6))
 (segment (start 93.98 161.896) (end 93.98 162.77) (width 0.4) (layer B.Cu) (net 6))
 (segment (start 71.12 154.94) (end 72.6586 154.94) (width 0.4) (layer B.Cu) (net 6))
 (segment (start 72.6586 154.94) (end 75.3132 152.285) (width 0.4) (layer B.Cu) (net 6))
 (segment (start 75.3132 152.285) (end 75.3132 147.34) (width 0.4) (layer B.Cu) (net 6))
 (segment (start 75.3132 147.34) (end 76.2795 146.374) (width 0.4) (layer B.Cu) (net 6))
 (segment (start 76.2795 146.374) (end 87.9538 146.374) (width 0.4) (layer B.Cu) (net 6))
 (segment (start 87.9538 146.374) (end 88.9 147.32) (width 0.4) (layer B.Cu) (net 6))
 (segment (start 88.9 147.32) (end 88.9 153.15) (width 0.4) (layer B.Cu) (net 6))
 (segment (start 99.06 153.15) (end 99.06 155.69) (width 0.4) (layer B.Cu) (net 7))
 (segment (start 99.06 155.69) (end 97.79 156.96) (width 0.4) (layer B.Cu) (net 7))
 (segment (start 97.79 156.96) (end 97.79 158.77) (width 0.4) (layer B.Cu) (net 7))
 (segment (start 101.6 162.77) (end 101.6 162.033) (width 0.4) (layer B.Cu) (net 7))
 (segment (start 101.6 162.033) (end 98.3367 158.77) (width 0.4) (layer B.Cu) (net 7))
 (segment (start 98.3367 158.77) (end 97.79 158.77) (width 0.4) (layer B.Cu) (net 7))
 (segment (start 99.06 153.15) (end 99.06 147.144) (width 0.4) (layer B.Cu) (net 7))
 (segment (start 99.06 147.144) (end 97.2768 145.361) (width 0.4) (layer B.Cu) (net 7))
 (segment (start 97.2768 145.361) (end 75.9942 145.361) (width 0.4) (layer B.Cu) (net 7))
 (segment (start 75.9942 145.361) (end 74.3408 147.015) (width 0.4) (layer B.Cu) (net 7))
 (segment (start 74.3408 147.015) (end 74.3408 150.729) (width 0.4) (layer B.Cu) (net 7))
 (segment (start 74.3408 150.729) (end 72.67 152.4) (width 0.4) (layer B.Cu) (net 7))
 (segment (start 72.67 152.4) (end 71.12 152.4) (width 0.4) (layer B.Cu) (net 7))
 (segment (start 109.22 153.15) (end 105.41 156.96) (width 0.4) (layer B.Cu) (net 8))
 (segment (start 105.41 156.96) (end 105.41 158.77) (width 0.4) (layer B.Cu) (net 8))
 (segment (start 105.41 158.77) (end 105.979 158.77) (width 0.4) (layer B.Cu) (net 8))
 (segment (start 105.979 158.77) (end 109.22 162.011) (width 0.4) (layer B.Cu) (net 8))
 (segment (start 109.22 162.011) (end 109.22 162.77) (width 0.4) (layer B.Cu) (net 8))
 (segment (start 109.22 153.15) (end 109.22 145.72) (width 0.4) (layer B.Cu) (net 8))
 (segment (start 109.22 145.72) (end 107.853 144.353) (width 0.4) (layer B.Cu) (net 8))
 (segment (start 107.853 144.353) (end 75.7879 144.353) (width 0.4) (layer B.Cu) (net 8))
 (segment (start 75.7879 144.353) (end 73.4921 146.648) (width 0.4) (layer B.Cu) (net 8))
 (segment (start 73.4921 146.648) (end 73.4921 150.028) (width 0.4) (layer B.Cu) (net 8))
 (segment (start 73.4921 150.028) (end 72.39 151.13) (width 0.4) (layer B.Cu) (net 8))
 (segment (start 72.39 151.13) (end 67.932 151.13) (width 0.4) (layer B.Cu) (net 8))
 (segment (start 67.932 151.13) (end 66.662 152.4) (width 0.4) (layer B.Cu) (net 8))
 (segment (start 66.662 152.4) (end 63.5 152.4) (width 0.4) (layer B.Cu) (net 8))
 (segment (start 90.17 166.37) (end 97.79 166.37) (width 0.4) (layer B.Cu) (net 4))
 (segment (start 90.17 162.77) (end 90.17 166.37) (width 0.4) (layer B.Cu) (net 4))
 (segment (start 106.68 141.2508) (end 106.68 141.901) (width 0.4) (layer B.Cu) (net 4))
 (segment (start 106.68 140.25) (end 106.68 141.2508) (width 0.4) (layer B.Cu) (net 4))
 (segment (start 97.79 166.37) (end 105.41 166.37) (width 0.4) (layer B.Cu) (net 4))
 (segment (start 53.34 149.275) (end 56.565 149.275) (width 0.4) (layer B.Cu) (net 4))
 (segment (start 56.565 149.275) (end 57.15 149.86) (width 0.4) (layer B.Cu) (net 4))
 (segment (start 48.26 149.275) (end 53.34 149.275) (width 0.4) (layer B.Cu) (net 4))
 (segment (start 57.15 149.86) (end 58.42 149.86) (width 0.4) (layer B.Cu) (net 4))
 (segment (start 58.42 149.86) (end 59.69 151.13) (width 0.4) (layer B.Cu) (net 4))
 (segment (start 59.69 151.13) (end 66.449 151.13) (width 0.4) (layer B.Cu) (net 4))
 (segment (start 66.449 151.13) (end 67.719 149.86) (width 0.4) (layer B.Cu) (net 4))
 (segment (start 67.719 149.86) (end 71.12 149.86) (width 0.4) (layer B.Cu) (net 4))
 (segment (start 71.12 149.86) (end 71.12 145.992) (width 0.4) (layer B.Cu) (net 4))
 (segment (start 71.12 145.992) (end 70.58 145.452) (width 0.4) (layer B.Cu) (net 4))
 (segment (start 70.58 145.452) (end 70.58 143.51) (width 0.4) (layer B.Cu) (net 4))
 (segment (start 53.34 150.4) (end 53.34 149.275) (width 0.4) (layer B.Cu) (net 4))
 (segment (start 97.79 141.901) (end 106.68 141.901) (width 0.4) (layer B.Cu) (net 4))
 (segment (start 70.58 143.51) (end 70.58 142.26) (width 0.4) (layer B.Cu) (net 4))
 (segment (start 70.58 142.26) (end 70.9389 141.901) (width 0.4) (layer B.Cu) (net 4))
 (segment (start 70.9389 141.901) (end 97.79 141.901) (width 0.4) (layer B.Cu) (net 4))
 (segment (start 96.99 133) (end 96.99 134.9) (width 0.4) (layer B.Cu) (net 4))
 (segment (start 96.99 134.9) (end 97.79 135.7) (width 0.4) (layer B.Cu) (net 4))
 (segment (start 97.79 135.7) (end 97.79 141.901) (width 0.4) (layer B.Cu) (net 4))
 (segment (start 105.41 166.37) (end 110.49 166.37) (width 0.4) (layer B.Cu) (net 4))
 (segment (start 110.49 166.37) (end 111.691 165.169) (width 0.4) (layer B.Cu) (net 4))
 (segment (start 111.691 165.169) (end 111.691 145.162) (width 0.4) (layer B.Cu) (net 4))
 (segment (start 111.691 145.162) (end 108.43 141.901) (width 0.4) (layer B.Cu) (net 4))
 (segment (start 108.43 141.901) (end 106.68 141.901) (width 0.4) (layer B.Cu) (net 4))
 (segment (start 105.41 162.77) (end 105.41 166.37) (width 0.4) (layer B.Cu) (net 4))
 (segment (start 97.79 162.77) (end 97.79 166.37) (width 0.4) (layer B.Cu) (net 4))
 (segment (start 82.55 162.77) (end 82.55 164.716) (width 0.4) (layer B.Cu) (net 4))
 (segment (start 82.55 164.716) (end 84.2043 166.37) (width 0.4) (layer B.Cu) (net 4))
 (segment (start 84.2043 166.37) (end 90.17 166.37) (width 0.4) (layer B.Cu) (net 4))
 (segment (start 48.26 149.275) (end 48.26 150.495) (width 0.4) (layer B.Cu) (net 4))
 (segment (start 48.26 149.275) (end 48.2694 149.266) (width 0.4) (layer B.Cu) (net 4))
 (segment (start 48.2694 149.266) (end 48.2694 145.742) (width 0.4) (layer B.Cu) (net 4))
 (segment (start 48.2694 145.742) (end 48.2694 149.266) (width 0.4) (layer F.Cu) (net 4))
 (segment (start 48.2694 149.266) (end 48.26 149.275) (width 0.4) (layer F.Cu) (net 4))
 (via (at 48.2694 145.742) (size 1) (layers F.Cu B.Cu) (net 4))
 (segment (start 63.5 160.02) (end 66.04 162.56) (width 0.4) (layer B.Cu) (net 9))
 (segment (start 62.96 159.48) (end 63.5 160.02) (width 0.4) (layer B.Cu) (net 9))
 (segment (start 63.5 160.02) (end 62.96 159.48) (width 0.4) (layer B.Cu) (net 9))
 (segment (start 65.8901 160.02) (end 63.5 160.02) (width 0.4) (layer B.Cu) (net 9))
 (segment (start 60.325 159.48) (end 62.96 159.48) (width 0.4) (layer B.Cu) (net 9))
 (segment (start 65.8901 160.02) (end 65.8901 162.41) (width 0.4) (layer B.Cu) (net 9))
 (segment (start 65.8901 162.41) (end 66.04 162.56) (width 0.4) (layer B.Cu) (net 9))
 (segment (start 60.325 155.48) (end 62.96 155.48) (width 0.4) (layer B.Cu) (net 3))
 (segment (start 62.96 155.48) (end 63.5 154.94) (width 0.4) (layer B.Cu) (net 3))
 (segment (start 60.325 155.33) (end 60.325 155.48) (width 0.4) (layer B.Cu) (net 3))
 (segment (start 57.15 152.4) (end 60.23 155.48) (width 0.4) (layer B.Cu) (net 3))
 (segment (start 60.23 155.48) (end 60.325 155.48) (width 0.4) (layer B.Cu) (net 3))
 (segment (start 66.04 146.05) (end 66.04 144.05) (width 0.4) (layer B.Cu) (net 10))
 (segment (start 66.04 144.05) (end 66.58 143.51) (width 0.4) (layer B.Cu) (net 10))
 (segment (start 63.5 149.86) (end 63.85 149.86) (width 0.4) (layer B.Cu) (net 10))
 (segment (start 63.85 149.86) (end 66.04 147.67) (width 0.4) (layer B.Cu) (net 10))
 (segment (start 66.04 147.67) (end 66.04 146.05) (width 0.4) (layer B.Cu) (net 10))
 (segment (start 63.425 149.86) (end 63.5 149.86) (width 0.4) (layer B.Cu) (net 10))
 (segment (start 57.15 157.48) (end 57.15 160.02) (width 0.4) (layer B.Cu) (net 1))
 (segment (start 57.15 160.02) (end 57.15 162.56) (width 0.4) (layer B.Cu) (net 1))
 (segment (start 106.68 135.7492) (end 106.68 135.099) (width 1) (layer B.Cu) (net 11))
 (segment (start 106.68 135.099) (end 109.901 135.099) (width 1) (layer B.Cu) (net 11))
 (segment (start 109.901 135.099) (end 113 132) (width 1) (layer B.Cu) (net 11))
 (segment (start 113 132) (end 119 132) (width 1) (layer B.Cu) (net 11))
 (segment (start 106.68 136.75) (end 106.68 135.7492) (width 1) (layer B.Cu) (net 11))
 (segment (start 117 120) (end 117 121.518) (width 1) (layer B.Cu) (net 11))
 (segment (start 117 121.518) (end 119 123.518) (width 1) (layer B.Cu) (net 11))
 (segment (start 119 123.518) (end 119 132) (width 1) (layer B.Cu) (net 11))
 (segment (start 119 132) (end 123 132) (width 1) (layer B.Cu) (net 11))
 (segment (start 124 146) (end 124 144.482) (width 1) (layer B.Cu) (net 11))
 (segment (start 124 144.482) (end 119 139.482) (width 1) (layer B.Cu) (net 11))
 (segment (start 119 139.482) (end 119 132) (width 1) (layer B.Cu) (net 11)))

